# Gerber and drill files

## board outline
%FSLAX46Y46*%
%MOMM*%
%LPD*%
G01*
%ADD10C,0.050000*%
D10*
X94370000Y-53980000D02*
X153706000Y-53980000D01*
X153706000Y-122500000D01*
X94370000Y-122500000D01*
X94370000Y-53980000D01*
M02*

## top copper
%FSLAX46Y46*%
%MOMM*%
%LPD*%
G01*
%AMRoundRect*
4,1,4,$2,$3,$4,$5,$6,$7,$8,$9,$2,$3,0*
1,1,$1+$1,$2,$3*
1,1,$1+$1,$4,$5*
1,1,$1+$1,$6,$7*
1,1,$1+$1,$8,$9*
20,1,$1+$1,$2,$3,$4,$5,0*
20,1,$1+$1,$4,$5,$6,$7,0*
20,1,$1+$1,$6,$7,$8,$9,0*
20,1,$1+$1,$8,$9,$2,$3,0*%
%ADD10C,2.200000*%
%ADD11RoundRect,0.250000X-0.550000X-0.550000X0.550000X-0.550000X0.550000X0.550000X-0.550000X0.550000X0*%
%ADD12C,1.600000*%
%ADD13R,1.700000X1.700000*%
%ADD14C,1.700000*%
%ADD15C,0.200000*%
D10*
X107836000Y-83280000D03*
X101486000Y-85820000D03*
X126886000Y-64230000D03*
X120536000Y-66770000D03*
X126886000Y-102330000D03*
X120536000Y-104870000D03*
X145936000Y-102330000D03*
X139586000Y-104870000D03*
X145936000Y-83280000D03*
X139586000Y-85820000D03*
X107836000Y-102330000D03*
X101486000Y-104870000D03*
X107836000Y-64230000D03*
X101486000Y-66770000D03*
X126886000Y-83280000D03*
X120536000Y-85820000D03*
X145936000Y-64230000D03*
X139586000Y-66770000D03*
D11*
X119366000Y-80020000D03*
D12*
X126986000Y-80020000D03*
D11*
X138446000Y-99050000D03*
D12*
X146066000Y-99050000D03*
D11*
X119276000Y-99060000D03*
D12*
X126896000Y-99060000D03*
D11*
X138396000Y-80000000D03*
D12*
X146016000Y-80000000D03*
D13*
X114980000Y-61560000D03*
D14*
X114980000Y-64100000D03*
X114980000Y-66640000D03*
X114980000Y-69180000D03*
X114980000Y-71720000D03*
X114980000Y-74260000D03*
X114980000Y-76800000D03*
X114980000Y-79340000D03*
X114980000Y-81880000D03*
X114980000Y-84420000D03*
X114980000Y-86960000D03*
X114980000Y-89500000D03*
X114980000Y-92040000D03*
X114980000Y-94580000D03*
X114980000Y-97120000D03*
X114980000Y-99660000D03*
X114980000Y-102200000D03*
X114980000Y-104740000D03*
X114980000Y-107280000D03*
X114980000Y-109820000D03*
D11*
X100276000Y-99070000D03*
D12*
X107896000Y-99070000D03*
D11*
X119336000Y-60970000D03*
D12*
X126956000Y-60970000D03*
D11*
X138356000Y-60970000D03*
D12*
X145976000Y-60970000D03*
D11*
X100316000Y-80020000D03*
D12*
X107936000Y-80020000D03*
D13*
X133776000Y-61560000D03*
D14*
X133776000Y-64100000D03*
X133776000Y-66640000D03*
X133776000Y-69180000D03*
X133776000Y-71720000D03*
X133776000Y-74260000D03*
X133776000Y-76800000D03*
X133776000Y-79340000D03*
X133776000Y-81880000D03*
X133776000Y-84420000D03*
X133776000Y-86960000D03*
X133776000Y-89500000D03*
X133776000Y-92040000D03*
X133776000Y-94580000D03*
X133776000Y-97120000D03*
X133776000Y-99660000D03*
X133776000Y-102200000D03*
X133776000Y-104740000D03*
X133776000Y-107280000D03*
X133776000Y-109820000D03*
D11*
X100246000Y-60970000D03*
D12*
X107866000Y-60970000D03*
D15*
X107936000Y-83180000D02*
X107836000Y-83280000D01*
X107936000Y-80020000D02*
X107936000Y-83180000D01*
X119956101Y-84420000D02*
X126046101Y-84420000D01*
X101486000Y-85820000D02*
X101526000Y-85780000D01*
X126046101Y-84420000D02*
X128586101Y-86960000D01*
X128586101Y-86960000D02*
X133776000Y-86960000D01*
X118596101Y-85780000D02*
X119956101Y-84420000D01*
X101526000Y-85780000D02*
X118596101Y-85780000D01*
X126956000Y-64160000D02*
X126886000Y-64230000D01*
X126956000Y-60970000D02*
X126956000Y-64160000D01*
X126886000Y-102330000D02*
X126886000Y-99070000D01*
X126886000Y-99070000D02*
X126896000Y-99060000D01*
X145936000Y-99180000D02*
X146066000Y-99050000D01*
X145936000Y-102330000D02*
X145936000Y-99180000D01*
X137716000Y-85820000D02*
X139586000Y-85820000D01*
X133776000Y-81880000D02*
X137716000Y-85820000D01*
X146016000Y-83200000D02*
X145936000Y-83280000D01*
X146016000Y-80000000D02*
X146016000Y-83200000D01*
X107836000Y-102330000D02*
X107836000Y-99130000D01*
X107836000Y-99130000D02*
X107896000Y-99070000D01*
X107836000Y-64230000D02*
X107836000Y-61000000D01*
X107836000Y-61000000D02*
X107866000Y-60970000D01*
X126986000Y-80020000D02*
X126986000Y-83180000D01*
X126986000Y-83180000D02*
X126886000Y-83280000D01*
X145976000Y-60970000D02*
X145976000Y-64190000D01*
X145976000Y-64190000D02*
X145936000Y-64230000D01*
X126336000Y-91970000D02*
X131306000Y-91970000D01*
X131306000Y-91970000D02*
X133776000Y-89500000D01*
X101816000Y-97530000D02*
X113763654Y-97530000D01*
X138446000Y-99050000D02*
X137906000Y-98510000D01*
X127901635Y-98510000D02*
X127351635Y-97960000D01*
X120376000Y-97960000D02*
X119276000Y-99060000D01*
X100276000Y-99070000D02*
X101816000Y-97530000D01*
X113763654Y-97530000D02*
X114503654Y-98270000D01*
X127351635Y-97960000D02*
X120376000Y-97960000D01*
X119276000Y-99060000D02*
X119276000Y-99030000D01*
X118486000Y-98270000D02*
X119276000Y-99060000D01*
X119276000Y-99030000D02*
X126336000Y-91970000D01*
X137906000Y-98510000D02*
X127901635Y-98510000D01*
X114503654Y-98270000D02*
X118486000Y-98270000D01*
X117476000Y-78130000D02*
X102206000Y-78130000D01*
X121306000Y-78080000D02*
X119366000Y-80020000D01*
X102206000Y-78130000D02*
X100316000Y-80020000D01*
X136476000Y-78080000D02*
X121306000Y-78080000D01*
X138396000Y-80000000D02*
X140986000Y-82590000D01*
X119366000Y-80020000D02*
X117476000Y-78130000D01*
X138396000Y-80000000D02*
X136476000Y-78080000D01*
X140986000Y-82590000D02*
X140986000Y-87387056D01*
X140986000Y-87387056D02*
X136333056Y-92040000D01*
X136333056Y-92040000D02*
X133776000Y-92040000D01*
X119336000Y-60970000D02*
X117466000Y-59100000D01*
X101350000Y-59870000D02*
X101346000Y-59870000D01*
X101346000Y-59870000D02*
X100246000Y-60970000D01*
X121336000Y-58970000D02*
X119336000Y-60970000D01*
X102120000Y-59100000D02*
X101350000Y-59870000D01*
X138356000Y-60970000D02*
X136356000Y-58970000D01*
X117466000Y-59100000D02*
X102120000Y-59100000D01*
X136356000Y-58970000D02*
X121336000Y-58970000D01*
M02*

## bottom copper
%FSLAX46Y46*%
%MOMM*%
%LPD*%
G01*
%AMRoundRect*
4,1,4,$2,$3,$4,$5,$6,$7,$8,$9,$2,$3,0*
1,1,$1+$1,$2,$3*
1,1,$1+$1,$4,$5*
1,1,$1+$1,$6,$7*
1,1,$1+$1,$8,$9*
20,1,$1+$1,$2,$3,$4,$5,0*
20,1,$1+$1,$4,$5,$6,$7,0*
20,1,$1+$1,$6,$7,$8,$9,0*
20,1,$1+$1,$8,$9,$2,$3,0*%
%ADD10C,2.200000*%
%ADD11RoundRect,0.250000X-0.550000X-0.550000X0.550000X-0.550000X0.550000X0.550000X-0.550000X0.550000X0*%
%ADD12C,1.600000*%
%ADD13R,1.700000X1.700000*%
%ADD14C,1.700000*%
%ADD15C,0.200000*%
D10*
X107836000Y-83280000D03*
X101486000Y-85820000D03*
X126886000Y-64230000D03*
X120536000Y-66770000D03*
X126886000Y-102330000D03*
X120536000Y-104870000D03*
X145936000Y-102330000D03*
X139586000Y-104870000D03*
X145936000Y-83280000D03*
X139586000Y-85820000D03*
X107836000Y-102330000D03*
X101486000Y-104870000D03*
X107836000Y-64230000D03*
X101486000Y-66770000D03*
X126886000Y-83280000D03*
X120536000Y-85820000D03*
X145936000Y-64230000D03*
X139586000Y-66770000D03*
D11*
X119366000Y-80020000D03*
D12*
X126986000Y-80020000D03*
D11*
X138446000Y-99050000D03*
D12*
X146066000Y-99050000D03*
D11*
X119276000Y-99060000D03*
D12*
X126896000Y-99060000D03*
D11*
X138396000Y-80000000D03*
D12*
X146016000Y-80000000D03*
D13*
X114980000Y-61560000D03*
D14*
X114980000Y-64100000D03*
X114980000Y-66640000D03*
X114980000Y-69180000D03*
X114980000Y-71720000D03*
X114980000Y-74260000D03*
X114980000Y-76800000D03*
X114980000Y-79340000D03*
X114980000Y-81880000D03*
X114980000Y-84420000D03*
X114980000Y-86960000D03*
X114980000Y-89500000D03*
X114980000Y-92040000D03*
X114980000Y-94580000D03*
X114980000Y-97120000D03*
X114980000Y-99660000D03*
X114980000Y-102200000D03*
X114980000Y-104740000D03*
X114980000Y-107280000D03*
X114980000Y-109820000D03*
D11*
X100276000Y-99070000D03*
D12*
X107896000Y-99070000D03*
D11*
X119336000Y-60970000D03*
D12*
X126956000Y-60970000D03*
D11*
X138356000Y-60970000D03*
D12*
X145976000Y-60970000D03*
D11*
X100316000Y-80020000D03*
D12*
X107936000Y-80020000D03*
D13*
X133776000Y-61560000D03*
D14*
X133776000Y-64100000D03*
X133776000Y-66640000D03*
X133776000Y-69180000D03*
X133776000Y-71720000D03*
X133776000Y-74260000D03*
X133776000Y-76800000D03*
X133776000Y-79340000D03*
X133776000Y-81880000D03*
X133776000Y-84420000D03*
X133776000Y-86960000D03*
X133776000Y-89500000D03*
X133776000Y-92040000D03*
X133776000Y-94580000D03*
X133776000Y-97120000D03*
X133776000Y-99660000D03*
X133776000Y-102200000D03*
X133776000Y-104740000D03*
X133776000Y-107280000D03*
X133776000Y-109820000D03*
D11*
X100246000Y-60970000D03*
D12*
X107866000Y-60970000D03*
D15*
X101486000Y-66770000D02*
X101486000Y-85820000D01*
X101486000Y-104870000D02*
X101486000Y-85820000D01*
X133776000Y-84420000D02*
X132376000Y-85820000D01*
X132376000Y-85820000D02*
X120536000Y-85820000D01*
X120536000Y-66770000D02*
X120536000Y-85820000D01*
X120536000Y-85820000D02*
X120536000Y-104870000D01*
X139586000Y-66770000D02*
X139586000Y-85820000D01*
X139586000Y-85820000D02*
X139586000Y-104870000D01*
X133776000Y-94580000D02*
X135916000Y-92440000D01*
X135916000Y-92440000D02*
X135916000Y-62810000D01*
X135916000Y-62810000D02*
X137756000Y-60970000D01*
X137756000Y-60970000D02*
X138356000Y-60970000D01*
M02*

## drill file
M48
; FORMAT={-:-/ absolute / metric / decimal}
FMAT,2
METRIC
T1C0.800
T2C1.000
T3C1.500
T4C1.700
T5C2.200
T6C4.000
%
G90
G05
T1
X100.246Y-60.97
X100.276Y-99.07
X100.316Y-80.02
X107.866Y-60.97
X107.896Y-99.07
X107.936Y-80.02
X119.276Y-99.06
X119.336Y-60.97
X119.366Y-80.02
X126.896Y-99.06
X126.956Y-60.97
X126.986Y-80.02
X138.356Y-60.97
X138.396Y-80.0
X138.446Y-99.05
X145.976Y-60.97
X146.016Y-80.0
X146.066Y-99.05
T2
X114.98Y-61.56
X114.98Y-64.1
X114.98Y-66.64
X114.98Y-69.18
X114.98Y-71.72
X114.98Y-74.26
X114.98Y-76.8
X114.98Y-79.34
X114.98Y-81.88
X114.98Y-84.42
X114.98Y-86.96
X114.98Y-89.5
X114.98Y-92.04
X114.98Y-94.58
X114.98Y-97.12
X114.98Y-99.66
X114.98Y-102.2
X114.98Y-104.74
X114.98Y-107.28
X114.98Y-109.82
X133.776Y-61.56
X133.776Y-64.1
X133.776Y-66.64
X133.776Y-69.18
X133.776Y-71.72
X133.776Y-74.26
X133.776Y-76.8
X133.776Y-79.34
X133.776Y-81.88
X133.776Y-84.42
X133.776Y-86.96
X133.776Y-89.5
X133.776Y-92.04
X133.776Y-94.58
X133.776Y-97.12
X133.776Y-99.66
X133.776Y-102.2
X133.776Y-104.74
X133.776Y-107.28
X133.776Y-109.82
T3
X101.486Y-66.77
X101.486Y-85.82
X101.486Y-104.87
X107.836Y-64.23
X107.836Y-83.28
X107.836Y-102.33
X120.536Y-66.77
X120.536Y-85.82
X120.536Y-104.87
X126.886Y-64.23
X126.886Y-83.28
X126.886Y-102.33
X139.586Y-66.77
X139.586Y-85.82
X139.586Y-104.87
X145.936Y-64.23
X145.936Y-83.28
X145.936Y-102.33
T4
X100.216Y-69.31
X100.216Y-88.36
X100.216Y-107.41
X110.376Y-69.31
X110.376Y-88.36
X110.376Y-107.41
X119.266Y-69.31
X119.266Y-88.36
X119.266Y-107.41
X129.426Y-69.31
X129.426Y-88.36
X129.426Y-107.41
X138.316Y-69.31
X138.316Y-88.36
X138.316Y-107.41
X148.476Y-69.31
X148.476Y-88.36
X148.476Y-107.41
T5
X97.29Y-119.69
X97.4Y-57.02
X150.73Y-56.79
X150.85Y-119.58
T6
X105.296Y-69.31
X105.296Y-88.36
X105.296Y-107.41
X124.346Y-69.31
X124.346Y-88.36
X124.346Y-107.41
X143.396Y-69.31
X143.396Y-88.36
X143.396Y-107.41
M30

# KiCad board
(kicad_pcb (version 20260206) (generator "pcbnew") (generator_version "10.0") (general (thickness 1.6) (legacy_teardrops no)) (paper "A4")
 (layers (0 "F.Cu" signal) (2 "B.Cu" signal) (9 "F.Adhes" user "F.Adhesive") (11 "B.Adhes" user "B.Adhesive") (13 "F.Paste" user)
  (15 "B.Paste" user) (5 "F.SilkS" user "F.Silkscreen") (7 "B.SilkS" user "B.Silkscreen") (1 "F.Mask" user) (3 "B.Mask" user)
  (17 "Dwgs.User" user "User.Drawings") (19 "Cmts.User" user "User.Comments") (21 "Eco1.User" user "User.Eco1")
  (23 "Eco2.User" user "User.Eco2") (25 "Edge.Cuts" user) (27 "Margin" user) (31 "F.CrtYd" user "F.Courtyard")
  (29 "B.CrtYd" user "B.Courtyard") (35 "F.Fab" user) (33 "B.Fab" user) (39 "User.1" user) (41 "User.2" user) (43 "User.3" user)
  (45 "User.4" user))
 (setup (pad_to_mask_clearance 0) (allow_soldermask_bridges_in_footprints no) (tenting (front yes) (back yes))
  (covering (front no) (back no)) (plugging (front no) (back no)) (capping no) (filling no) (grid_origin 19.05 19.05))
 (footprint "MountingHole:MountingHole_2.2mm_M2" (layer "F.Cu") (at 150.73 56.79)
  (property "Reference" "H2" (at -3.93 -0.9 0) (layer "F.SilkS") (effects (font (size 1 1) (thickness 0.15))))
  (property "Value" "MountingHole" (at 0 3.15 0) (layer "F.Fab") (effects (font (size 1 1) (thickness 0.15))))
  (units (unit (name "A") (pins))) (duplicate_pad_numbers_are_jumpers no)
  (pad "" np_thru_hole circle (at 0 0) (size 2.2 2.2) (drill 2.2) (layers "*.Cu" "*.Mask")))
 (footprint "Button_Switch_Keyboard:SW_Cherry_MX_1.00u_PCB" (layer "F.Cu") (at 107.836 83.28)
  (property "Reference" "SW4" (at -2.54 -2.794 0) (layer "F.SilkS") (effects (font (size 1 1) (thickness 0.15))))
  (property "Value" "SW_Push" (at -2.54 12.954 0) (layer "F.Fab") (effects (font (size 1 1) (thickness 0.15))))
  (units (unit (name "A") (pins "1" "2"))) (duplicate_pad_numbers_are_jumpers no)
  (pad "" np_thru_hole circle (at -7.62 5.08) (size 1.7 1.7) (drill 1.7) (layers "*.Cu" "*.Mask"))
  (pad "" np_thru_hole circle (at -2.54 5.08) (size 4 4) (drill 4) (layers "*.Cu" "*.Mask"))
  (pad "" np_thru_hole circle (at 2.54 5.08) (size 1.7 1.7) (drill 1.7) (layers "*.Cu" "*.Mask"))
  (pad "1" thru_hole circle (at 0 0) (size 2.2 2.2) (drill 1.5) (layers "*.Cu" "*.Mask") (remove_unused_layers no) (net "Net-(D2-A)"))
  (pad "2" thru_hole circle (at -6.35 2.54) (size 2.2 2.2) (drill 1.5) (layers "*.Cu" "*.Mask") (remove_unused_layers no) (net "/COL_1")))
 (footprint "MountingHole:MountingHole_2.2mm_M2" (layer "F.Cu") (at 97.4 57.02)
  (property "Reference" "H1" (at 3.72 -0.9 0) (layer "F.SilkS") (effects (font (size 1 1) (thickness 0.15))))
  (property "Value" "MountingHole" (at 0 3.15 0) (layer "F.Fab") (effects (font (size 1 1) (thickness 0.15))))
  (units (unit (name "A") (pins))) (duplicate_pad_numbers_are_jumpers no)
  (pad "" np_thru_hole circle (at 0 0) (size 2.2 2.2) (drill 2.2) (layers "*.Cu" "*.Mask")))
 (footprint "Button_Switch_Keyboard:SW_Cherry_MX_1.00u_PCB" (layer "F.Cu") (at 126.886 64.23)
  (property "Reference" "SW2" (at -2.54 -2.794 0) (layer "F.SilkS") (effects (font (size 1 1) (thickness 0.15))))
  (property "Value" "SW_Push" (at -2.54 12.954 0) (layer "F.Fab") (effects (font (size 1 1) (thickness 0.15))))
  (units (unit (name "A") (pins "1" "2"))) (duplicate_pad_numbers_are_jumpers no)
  (pad "" np_thru_hole circle (at -7.62 5.08) (size 1.7 1.7) (drill 1.7) (layers "*.Cu" "*.Mask"))
  (pad "" np_thru_hole circle (at -2.54 5.08) (size 4 4) (drill 4) (layers "*.Cu" "*.Mask"))
  (pad "" np_thru_hole circle (at 2.54 5.08) (size 1.7 1.7) (drill 1.7) (layers "*.Cu" "*.Mask"))
  (pad "1" thru_hole circle (at 0 0) (size 2.2 2.2) (drill 1.5) (layers "*.Cu" "*.Mask") (remove_unused_layers no) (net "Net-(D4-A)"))
  (pad "2" thru_hole circle (at -6.35 2.54) (size 2.2 2.2) (drill 1.5) (layers "*.Cu" "*.Mask") (remove_unused_layers no) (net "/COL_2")))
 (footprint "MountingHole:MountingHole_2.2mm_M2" (layer "F.Cu") (at 97.29 119.69)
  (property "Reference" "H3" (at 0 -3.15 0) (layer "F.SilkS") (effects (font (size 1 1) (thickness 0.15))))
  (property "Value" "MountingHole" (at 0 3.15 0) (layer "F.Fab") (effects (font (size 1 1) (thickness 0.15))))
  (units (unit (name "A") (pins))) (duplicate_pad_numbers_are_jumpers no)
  (pad "" np_thru_hole circle (at 0 0) (size 2.2 2.2) (drill 2.2) (layers "*.Cu" "*.Mask")))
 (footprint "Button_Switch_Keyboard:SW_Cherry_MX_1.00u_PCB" (layer "F.Cu") (at 126.886 102.33)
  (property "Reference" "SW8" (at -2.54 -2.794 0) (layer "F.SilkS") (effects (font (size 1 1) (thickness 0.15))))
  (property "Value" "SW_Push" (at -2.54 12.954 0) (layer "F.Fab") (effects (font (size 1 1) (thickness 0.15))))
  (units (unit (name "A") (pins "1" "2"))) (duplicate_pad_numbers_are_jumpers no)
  (pad "" np_thru_hole circle (at -7.62 5.08) (size 1.7 1.7) (drill 1.7) (layers "*.Cu" "*.Mask"))
  (pad "" np_thru_hole circle (at -2.54 5.08) (size 4 4) (drill 4) (layers "*.Cu" "*.Mask"))
  (pad "" np_thru_hole circle (at 2.54 5.08) (size 1.7 1.7) (drill 1.7) (layers "*.Cu" "*.Mask"))
  (pad "1" thru_hole circle (at 0 0) (size 2.2 2.2) (drill 1.5) (layers "*.Cu" "*.Mask") (remove_unused_layers no) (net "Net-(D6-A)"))
  (pad "2" thru_hole circle (at -6.35 2.54) (size 2.2 2.2) (drill 1.5) (layers "*.Cu" "*.Mask") (remove_unused_layers no) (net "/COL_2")))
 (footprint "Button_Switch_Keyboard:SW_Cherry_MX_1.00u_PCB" (layer "F.Cu") (at 145.936 102.33)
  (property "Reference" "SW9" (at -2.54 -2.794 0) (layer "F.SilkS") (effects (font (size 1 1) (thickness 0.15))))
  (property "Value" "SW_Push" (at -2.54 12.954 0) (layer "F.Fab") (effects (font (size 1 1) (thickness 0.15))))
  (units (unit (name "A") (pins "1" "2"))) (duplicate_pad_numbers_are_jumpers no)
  (pad "" np_thru_hole circle (at -7.62 5.08) (size 1.7 1.7) (drill 1.7) (layers "*.Cu" "*.Mask"))
  (pad "" np_thru_hole circle (at -2.54 5.08) (size 4 4) (drill 4) (layers "*.Cu" "*.Mask"))
  (pad "" np_thru_hole circle (at 2.54 5.08) (size 1.7 1.7) (drill 1.7) (layers "*.Cu" "*.Mask"))
  (pad "1" thru_hole circle (at 0 0) (size 2.2 2.2) (drill 1.5) (layers "*.Cu" "*.Mask") (remove_unused_layers no) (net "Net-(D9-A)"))
  (pad "2" thru_hole circle (at -6.35 2.54) (size 2.2 2.2) (drill 1.5) (layers "*.Cu" "*.Mask") (remove_unused_layers no) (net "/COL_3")))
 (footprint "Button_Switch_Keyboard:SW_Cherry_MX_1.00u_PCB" (layer "F.Cu") (at 145.936 83.28)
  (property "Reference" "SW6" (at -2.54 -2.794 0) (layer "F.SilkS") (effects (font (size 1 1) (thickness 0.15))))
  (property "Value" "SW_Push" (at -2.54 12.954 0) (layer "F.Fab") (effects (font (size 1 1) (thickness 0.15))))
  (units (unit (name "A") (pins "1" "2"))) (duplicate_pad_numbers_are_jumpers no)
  (pad "" np_thru_hole circle (at -7.62 5.08) (size 1.7 1.7) (drill 1.7) (layers "*.Cu" "*.Mask"))
  (pad "" np_thru_hole circle (at -2.54 5.08) (size 4 4) (drill 4) (layers "*.Cu" "*.Mask"))
  (pad "" np_thru_hole circle (at 2.54 5.08) (size 1.7 1.7) (drill 1.7) (layers "*.Cu" "*.Mask"))
  (pad "1" thru_hole circle (at 0 0) (size 2.2 2.2) (drill 1.5) (layers "*.Cu" "*.Mask") (remove_unused_layers no) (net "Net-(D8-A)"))
  (pad "2" thru_hole circle (at -6.35 2.54) (size 2.2 2.2) (drill 1.5) (layers "*.Cu" "*.Mask") (remove_unused_layers no) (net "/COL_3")))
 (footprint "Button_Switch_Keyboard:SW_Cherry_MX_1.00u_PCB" (layer "F.Cu") (at 107.836 102.33)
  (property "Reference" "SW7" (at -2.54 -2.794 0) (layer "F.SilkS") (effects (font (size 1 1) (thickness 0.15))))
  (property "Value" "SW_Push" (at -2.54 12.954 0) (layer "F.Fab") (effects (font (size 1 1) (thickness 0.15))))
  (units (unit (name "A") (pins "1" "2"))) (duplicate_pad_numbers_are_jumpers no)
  (pad "" np_thru_hole circle (at -7.62 5.08) (size 1.7 1.7) (drill 1.7) (layers "*.Cu" "*.Mask"))
  (pad "" np_thru_hole circle (at -2.54 5.08) (size 4 4) (drill 4) (layers "*.Cu" "*.Mask"))
  (pad "" np_thru_hole circle (at 2.54 5.08) (size 1.7 1.7) (drill 1.7) (layers "*.Cu" "*.Mask"))
  (pad "1" thru_hole circle (at 0 0) (size 2.2 2.2) (drill 1.5) (layers "*.Cu" "*.Mask") (remove_unused_layers no) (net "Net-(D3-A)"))
  (pad "2" thru_hole circle (at -6.35 2.54) (size 2.2 2.2) (drill 1.5) (layers "*.Cu" "*.Mask") (remove_unused_layers no) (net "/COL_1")))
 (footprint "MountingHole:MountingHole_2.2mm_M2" (layer "F.Cu") (at 150.85 119.58)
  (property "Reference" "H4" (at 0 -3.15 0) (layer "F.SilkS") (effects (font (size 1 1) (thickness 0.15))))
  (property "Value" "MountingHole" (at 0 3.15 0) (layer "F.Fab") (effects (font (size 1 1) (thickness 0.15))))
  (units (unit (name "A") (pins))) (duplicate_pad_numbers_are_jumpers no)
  (pad "" np_thru_hole circle (at 0 0) (size 2.2 2.2) (drill 2.2) (layers "*.Cu" "*.Mask")))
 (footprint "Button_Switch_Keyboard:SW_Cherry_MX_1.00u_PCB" (layer "F.Cu") (at 107.836 64.23)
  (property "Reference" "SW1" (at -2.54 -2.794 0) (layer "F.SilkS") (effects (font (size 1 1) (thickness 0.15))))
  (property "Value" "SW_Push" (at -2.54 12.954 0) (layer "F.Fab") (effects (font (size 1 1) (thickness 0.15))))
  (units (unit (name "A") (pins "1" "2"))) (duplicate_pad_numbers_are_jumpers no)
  (pad "" np_thru_hole circle (at -7.62 5.08) (size 1.7 1.7) (drill 1.7) (layers "*.Cu" "*.Mask"))
  (pad "" np_thru_hole circle (at -2.54 5.08) (size 4 4) (drill 4) (layers "*.Cu" "*.Mask"))
  (pad "" np_thru_hole circle (at 2.54 5.08) (size 1.7 1.7) (drill 1.7) (layers "*.Cu" "*.Mask"))
  (pad "1" thru_hole circle (at 0 0) (size 2.2 2.2) (drill 1.5) (layers "*.Cu" "*.Mask") (remove_unused_layers no) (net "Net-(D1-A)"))
  (pad "2" thru_hole circle (at -6.35 2.54) (size 2.2 2.2) (drill 1.5) (layers "*.Cu" "*.Mask") (remove_unused_layers no) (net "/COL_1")))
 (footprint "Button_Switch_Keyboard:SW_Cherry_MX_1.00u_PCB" (layer "F.Cu") (at 126.886 83.28)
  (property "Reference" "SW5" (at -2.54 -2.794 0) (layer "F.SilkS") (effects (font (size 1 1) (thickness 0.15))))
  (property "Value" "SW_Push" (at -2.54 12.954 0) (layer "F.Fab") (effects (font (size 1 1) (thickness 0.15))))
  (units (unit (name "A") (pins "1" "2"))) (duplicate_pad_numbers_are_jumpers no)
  (pad "" np_thru_hole circle (at -7.62 5.08) (size 1.7 1.7) (drill 1.7) (layers "*.Cu" "*.Mask"))
  (pad "" np_thru_hole circle (at -2.54 5.08) (size 4 4) (drill 4) (layers "*.Cu" "*.Mask"))
  (pad "" np_thru_hole circle (at 2.54 5.08) (size 1.7 1.7) (drill 1.7) (layers "*.Cu" "*.Mask"))
  (pad "1" thru_hole circle (at 0 0) (size 2.2 2.2) (drill 1.5) (layers "*.Cu" "*.Mask") (remove_unused_layers no) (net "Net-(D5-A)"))
  (pad "2" thru_hole circle (at -6.35 2.54) (size 2.2 2.2) (drill 1.5) (layers "*.Cu" "*.Mask") (remove_unused_layers no) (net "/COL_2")))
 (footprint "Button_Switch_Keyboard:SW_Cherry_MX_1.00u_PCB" (layer "F.Cu") (at 145.936 64.23)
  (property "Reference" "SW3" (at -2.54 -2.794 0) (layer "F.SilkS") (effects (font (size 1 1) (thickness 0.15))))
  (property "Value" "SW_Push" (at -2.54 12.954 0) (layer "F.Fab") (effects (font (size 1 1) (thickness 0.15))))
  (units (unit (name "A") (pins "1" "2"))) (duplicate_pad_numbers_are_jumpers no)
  (pad "" np_thru_hole circle (at -7.62 5.08) (size 1.7 1.7) (drill 1.7) (layers "*.Cu" "*.Mask"))
  (pad "" np_thru_hole circle (at -2.54 5.08) (size 4 4) (drill 4) (layers "*.Cu" "*.Mask"))
  (pad "" np_thru_hole circle (at 2.54 5.08) (size 1.7 1.7) (drill 1.7) (layers "*.Cu" "*.Mask"))
  (pad "1" thru_hole circle (at 0 0) (size 2.2 2.2) (drill 1.5) (layers "*.Cu" "*.Mask") (remove_unused_layers no) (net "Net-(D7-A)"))
  (pad "2" thru_hole circle (at -6.35 2.54) (size 2.2 2.2) (drill 1.5) (layers "*.Cu" "*.Mask") (remove_unused_layers no) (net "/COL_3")))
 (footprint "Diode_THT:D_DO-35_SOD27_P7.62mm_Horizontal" (layer "B.Cu") (at 119.366 80.02)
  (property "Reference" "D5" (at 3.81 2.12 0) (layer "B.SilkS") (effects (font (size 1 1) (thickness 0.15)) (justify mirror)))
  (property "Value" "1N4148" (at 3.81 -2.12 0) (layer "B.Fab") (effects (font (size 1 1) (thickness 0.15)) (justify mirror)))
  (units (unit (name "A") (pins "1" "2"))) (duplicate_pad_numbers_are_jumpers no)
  (pad "1" thru_hole roundrect (at 0 0) (size 1.6 1.6) (drill 0.8) (layers "*.Cu" "*.Mask") (remove_unused_layers no)
   (roundrect_rratio 0.15625) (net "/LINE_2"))
  (pad "2" thru_hole circle (at 7.62 0) (size 1.6 1.6) (drill 0.8) (layers "*.Cu" "*.Mask") (remove_unused_layers no) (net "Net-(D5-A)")))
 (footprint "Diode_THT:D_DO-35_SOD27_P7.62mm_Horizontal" (layer "B.Cu") (at 138.446 99.05)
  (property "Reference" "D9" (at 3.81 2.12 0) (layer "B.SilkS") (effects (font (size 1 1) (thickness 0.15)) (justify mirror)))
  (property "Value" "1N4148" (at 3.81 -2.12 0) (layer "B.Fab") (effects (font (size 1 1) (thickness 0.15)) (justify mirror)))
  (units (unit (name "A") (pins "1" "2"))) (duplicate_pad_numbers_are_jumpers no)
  (pad "1" thru_hole roundrect (at 0 0) (size 1.6 1.6) (drill 0.8) (layers "*.Cu" "*.Mask") (remove_unused_layers no)
   (roundrect_rratio 0.15625) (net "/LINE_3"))
  (pad "2" thru_hole circle (at 7.62 0) (size 1.6 1.6) (drill 0.8) (layers "*.Cu" "*.Mask") (remove_unused_layers no) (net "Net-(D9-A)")))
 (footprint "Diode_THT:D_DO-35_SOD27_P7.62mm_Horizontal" (layer "B.Cu") (at 119.276 99.06)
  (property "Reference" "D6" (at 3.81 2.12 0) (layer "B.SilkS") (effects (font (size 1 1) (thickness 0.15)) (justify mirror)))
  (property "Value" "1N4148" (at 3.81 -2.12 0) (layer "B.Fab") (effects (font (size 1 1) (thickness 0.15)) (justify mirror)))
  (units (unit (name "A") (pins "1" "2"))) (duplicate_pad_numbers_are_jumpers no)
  (pad "1" thru_hole roundrect (at 0 0) (size 1.6 1.6) (drill 0.8) (layers "*.Cu" "*.Mask") (remove_unused_layers no)
   (roundrect_rratio 0.15625) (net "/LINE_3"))
  (pad "2" thru_hole circle (at 7.62 0) (size 1.6 1.6) (drill 0.8) (layers "*.Cu" "*.Mask") (remove_unused_layers no) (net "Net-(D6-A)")))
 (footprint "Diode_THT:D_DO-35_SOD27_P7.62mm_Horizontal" (layer "B.Cu") (at 138.396 80)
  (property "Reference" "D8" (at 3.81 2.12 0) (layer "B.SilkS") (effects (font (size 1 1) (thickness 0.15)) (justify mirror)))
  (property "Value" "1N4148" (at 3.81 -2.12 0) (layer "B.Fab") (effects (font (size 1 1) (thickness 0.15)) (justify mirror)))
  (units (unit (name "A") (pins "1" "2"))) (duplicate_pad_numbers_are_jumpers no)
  (pad "1" thru_hole roundrect (at 0 0) (size 1.6 1.6) (drill 0.8) (layers "*.Cu" "*.Mask") (remove_unused_layers no)
   (roundrect_rratio 0.15625) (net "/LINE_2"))
  (pad "2" thru_hole circle (at 7.62 0) (size 1.6 1.6) (drill 0.8) (layers "*.Cu" "*.Mask") (remove_unused_layers no) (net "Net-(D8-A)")))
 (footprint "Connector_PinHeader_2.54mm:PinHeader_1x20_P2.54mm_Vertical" (layer "B.Cu") (at 114.98 61.56 180)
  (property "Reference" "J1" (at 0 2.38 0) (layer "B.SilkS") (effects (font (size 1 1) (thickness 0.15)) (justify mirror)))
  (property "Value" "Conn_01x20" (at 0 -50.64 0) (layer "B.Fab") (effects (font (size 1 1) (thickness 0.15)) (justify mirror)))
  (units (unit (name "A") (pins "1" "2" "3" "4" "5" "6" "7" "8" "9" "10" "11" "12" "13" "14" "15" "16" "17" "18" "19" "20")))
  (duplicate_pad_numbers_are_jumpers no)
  (pad "1" thru_hole rect (at 0 0 180) (size 1.7 1.7) (drill 1) (layers "*.Cu" "*.Mask") (remove_unused_layers no)
   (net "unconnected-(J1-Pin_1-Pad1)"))
  (pad "2" thru_hole circle (at 0 -2.54 180) (size 1.7 1.7) (drill 1) (layers "*.Cu" "*.Mask") (remove_unused_layers no)
   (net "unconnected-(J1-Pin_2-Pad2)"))
  (pad "3" thru_hole circle (at 0 -5.08 180) (size 1.7 1.7) (drill 1) (layers "*.Cu" "*.Mask") (remove_unused_layers no)
   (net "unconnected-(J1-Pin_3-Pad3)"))
  (pad "4" thru_hole circle (at 0 -7.62 180) (size 1.7 1.7) (drill 1) (layers "*.Cu" "*.Mask") (remove_unused_layers no)
   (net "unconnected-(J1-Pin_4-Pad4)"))
  (pad "5" thru_hole circle (at 0 -10.16 180) (size 1.7 1.7) (drill 1) (layers "*.Cu" "*.Mask") (remove_unused_layers no)
   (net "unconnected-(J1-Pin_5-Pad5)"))
  (pad "6" thru_hole circle (at 0 -12.7 180) (size 1.7 1.7) (drill 1) (layers "*.Cu" "*.Mask") (remove_unused_layers no)
   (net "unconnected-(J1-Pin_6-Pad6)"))
  (pad "7" thru_hole circle (at 0 -15.24 180) (size 1.7 1.7) (drill 1) (layers "*.Cu" "*.Mask") (remove_unused_layers no)
   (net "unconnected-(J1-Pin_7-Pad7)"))
  (pad "8" thru_hole circle (at 0 -17.78 180) (size 1.7 1.7) (drill 1) (layers "*.Cu" "*.Mask") (remove_unused_layers no)
   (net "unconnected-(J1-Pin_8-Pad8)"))
  (pad "9" thru_hole circle (at 0 -20.32 180) (size 1.7 1.7) (drill 1) (layers "*.Cu" "*.Mask") (remove_unused_layers no)
   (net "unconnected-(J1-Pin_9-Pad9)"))
  (pad "10" thru_hole circle (at 0 -22.86 180) (size 1.7 1.7) (drill 1) (layers "*.Cu" "*.Mask") (remove_unused_layers no)
   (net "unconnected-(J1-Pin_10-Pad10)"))
  (pad "11" thru_hole circle (at 0 -25.4 180) (size 1.7 1.7) (drill 1) (layers "*.Cu" "*.Mask") (remove_unused_layers no)
   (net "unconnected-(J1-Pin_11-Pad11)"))
  (pad "12" thru_hole circle (at 0 -27.94 180) (size 1.7 1.7) (drill 1) (layers "*.Cu" "*.Mask") (remove_unused_layers no)
   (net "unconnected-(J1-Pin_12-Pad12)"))
  (pad "13" thru_hole circle (at 0 -30.48 180) (size 1.7 1.7) (drill 1) (layers "*.Cu" "*.Mask") (remove_unused_layers no)
   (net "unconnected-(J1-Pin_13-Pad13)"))
  (pad "14" thru_hole circle (at 0 -33.02 180) (size 1.7 1.7) (drill 1) (layers "*.Cu" "*.Mask") (remove_unused_layers no)
   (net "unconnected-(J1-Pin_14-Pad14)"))
  (pad "15" thru_hole circle (at 0 -35.56 180) (size 1.7 1.7) (drill 1) (layers "*.Cu" "*.Mask") (remove_unused_layers no)
   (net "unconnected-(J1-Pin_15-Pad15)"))
  (pad "16" thru_hole circle (at 0 -38.1 180) (size 1.7 1.7) (drill 1) (layers "*.Cu" "*.Mask") (remove_unused_layers no)
   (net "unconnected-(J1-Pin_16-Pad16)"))
  (pad "17" thru_hole circle (at 0 -40.64 180) (size 1.7 1.7) (drill 1) (layers "*.Cu" "*.Mask") (remove_unused_layers no)
   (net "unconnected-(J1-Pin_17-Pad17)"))
  (pad "18" thru_hole circle (at 0 -43.18 180) (size 1.7 1.7) (drill 1) (layers "*.Cu" "*.Mask") (remove_unused_layers no)
   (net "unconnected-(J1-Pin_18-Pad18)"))
  (pad "19" thru_hole circle (at 0 -45.72 180) (size 1.7 1.7) (drill 1) (layers "*.Cu" "*.Mask") (remove_unused_layers no)
   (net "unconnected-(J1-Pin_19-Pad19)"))
  (pad "20" thru_hole circle (at 0 -48.26 180) (size 1.7 1.7) (drill 1) (layers "*.Cu" "*.Mask") (remove_unused_layers no)
   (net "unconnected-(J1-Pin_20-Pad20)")))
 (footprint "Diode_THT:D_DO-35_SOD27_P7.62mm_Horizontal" (layer "B.Cu") (at 100.276 99.07)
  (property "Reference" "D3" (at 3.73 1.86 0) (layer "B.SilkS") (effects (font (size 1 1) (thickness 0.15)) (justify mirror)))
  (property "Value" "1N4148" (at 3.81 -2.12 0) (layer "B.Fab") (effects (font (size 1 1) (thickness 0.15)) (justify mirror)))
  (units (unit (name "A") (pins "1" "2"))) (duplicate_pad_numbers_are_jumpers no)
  (pad "1" thru_hole roundrect (at 0 0) (size 1.6 1.6) (drill 0.8) (layers "*.Cu" "*.Mask") (remove_unused_layers no)
   (roundrect_rratio 0.15625) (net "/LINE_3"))
  (pad "2" thru_hole circle (at 7.62 0) (size 1.6 1.6) (drill 0.8) (layers "*.Cu" "*.Mask") (remove_unused_layers no) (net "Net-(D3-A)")))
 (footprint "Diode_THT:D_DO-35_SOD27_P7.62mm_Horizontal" (layer "B.Cu") (at 119.336 60.97)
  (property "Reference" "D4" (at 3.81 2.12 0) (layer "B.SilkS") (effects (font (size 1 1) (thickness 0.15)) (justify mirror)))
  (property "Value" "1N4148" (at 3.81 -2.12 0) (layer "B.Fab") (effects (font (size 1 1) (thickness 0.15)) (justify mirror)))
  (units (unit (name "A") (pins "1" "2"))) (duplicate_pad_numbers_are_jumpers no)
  (pad "1" thru_hole roundrect (at 0 0) (size 1.6 1.6) (drill 0.8) (layers "*.Cu" "*.Mask") (remove_unused_layers no)
   (roundrect_rratio 0.15625) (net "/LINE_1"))
  (pad "2" thru_hole circle (at 7.62 0) (size 1.6 1.6) (drill 0.8) (layers "*.Cu" "*.Mask") (remove_unused_layers no) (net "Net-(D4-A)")))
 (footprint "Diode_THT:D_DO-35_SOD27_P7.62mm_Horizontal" (layer "B.Cu") (at 138.356 60.97)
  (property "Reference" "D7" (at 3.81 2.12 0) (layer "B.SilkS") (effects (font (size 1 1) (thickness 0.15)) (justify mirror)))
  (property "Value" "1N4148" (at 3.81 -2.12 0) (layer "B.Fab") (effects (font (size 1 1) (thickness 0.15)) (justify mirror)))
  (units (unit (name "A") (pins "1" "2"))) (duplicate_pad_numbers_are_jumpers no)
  (pad "1" thru_hole roundrect (at 0 0) (size 1.6 1.6) (drill 0.8) (layers "*.Cu" "*.Mask") (remove_unused_layers no)
   (roundrect_rratio 0.15625) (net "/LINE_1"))
  (pad "2" thru_hole circle (at 7.62 0) (size 1.6 1.6) (drill 0.8) (layers "*.Cu" "*.Mask") (remove_unused_layers no) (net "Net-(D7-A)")))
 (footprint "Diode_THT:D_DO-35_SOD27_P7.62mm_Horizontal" (layer "B.Cu") (at 100.316 80.02)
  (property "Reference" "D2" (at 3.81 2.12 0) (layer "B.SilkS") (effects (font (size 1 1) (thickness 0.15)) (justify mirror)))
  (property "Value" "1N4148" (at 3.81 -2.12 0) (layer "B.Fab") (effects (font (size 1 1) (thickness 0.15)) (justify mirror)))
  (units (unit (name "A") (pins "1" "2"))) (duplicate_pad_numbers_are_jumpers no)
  (pad "1" thru_hole roundrect (at 0 0) (size 1.6 1.6) (drill 0.8) (layers "*.Cu" "*.Mask") (remove_unused_layers no)
   (roundrect_rratio 0.15625) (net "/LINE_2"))
  (pad "2" thru_hole circle (at 7.62 0) (size 1.6 1.6) (drill 0.8) (layers "*.Cu" "*.Mask") (remove_unused_layers no) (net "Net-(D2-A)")))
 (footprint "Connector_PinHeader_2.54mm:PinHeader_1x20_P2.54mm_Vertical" (layer "B.Cu") (at 133.776 61.56 180)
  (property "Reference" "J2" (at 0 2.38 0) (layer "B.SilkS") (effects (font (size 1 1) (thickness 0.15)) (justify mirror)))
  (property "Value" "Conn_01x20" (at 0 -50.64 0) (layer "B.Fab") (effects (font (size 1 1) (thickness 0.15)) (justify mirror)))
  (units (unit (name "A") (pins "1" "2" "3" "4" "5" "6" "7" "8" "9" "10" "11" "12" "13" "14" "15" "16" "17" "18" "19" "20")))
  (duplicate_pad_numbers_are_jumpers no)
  (pad "1" thru_hole rect (at 0 0 180) (size 1.7 1.7) (drill 1) (layers "*.Cu" "*.Mask") (remove_unused_layers no)
   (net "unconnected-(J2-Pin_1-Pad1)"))
  (pad "2" thru_hole circle (at 0 -2.54 180) (size 1.7 1.7) (drill 1) (layers "*.Cu" "*.Mask") (remove_unused_layers no)
   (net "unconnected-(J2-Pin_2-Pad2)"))
  (pad "3" thru_hole circle (at 0 -5.08 180) (size 1.7 1.7) (drill 1) (layers "*.Cu" "*.Mask") (remove_unused_layers no)
   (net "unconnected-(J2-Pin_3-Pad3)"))
  (pad "4" thru_hole circle (at 0 -7.62 180) (size 1.7 1.7) (drill 1) (layers "*.Cu" "*.Mask") (remove_unused_layers no)
   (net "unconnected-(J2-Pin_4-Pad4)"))
  (pad "5" thru_hole circle (at 0 -10.16 180) (size 1.7 1.7) (drill 1) (layers "*.Cu" "*.Mask") (remove_unused_layers no)
   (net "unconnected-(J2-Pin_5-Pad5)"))
  (pad "6" thru_hole circle (at 0 -12.7 180) (size 1.7 1.7) (drill 1) (layers "*.Cu" "*.Mask") (remove_unused_layers no)
   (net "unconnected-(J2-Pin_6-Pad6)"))
  (pad "7" thru_hole circle (at 0 -15.24 180) (size 1.7 1.7) (drill 1) (layers "*.Cu" "*.Mask") (remove_unused_layers no)
   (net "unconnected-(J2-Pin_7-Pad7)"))
  (pad "8" thru_hole circle (at 0 -17.78 180) (size 1.7 1.7) (drill 1) (layers "*.Cu" "*.Mask") (remove_unused_layers no)
   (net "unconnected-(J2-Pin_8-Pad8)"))
  (pad "9" thru_hole circle (at 0 -20.32 180) (size 1.7 1.7) (drill 1) (layers "*.Cu" "*.Mask") (remove_unused_layers no) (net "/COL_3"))
  (pad "10" thru_hole circle (at 0 -22.86 180) (size 1.7 1.7) (drill 1) (layers "*.Cu" "*.Mask") (remove_unused_layers no) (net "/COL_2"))
  (pad "11" thru_hole circle (at 0 -25.4 180) (size 1.7 1.7) (drill 1) (layers "*.Cu" "*.Mask") (remove_unused_layers no) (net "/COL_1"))
  (pad "12" thru_hole circle (at 0 -27.94 180) (size 1.7 1.7) (drill 1) (layers "*.Cu" "*.Mask") (remove_unused_layers no) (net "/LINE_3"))
  (pad "13" thru_hole circle (at 0 -30.48 180) (size 1.7 1.7) (drill 1) (layers "*.Cu" "*.Mask") (remove_unused_layers no) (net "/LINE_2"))
  (pad "14" thru_hole circle (at 0 -33.02 180) (size 1.7 1.7) (drill 1) (layers "*.Cu" "*.Mask") (remove_unused_layers no) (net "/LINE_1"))
  (pad "15" thru_hole circle (at 0 -35.56 180) (size 1.7 1.7) (drill 1) (layers "*.Cu" "*.Mask") (remove_unused_layers no)
   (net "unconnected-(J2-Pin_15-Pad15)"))
  (pad "16" thru_hole circle (at 0 -38.1 180) (size 1.7 1.7) (drill 1) (layers "*.Cu" "*.Mask") (remove_unused_layers no)
   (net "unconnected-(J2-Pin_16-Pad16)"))
  (pad "17" thru_hole circle (at 0 -40.64 180) (size 1.7 1.7) (drill 1) (layers "*.Cu" "*.Mask") (remove_unused_layers no)
   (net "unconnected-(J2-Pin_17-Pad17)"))
  (pad "18" thru_hole circle (at 0 -43.18 180) (size 1.7 1.7) (drill 1) (layers "*.Cu" "*.Mask") (remove_unused_layers no)
   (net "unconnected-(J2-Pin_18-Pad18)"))
  (pad "19" thru_hole circle (at 0 -45.72 180) (size 1.7 1.7) (drill 1) (layers "*.Cu" "*.Mask") (remove_unused_layers no)
   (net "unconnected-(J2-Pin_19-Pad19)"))
  (pad "20" thru_hole circle (at 0 -48.26 180) (size 1.7 1.7) (drill 1) (layers "*.Cu" "*.Mask") (remove_unused_layers no)
   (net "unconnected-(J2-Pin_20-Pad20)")))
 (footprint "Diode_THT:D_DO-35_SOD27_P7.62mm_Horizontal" (layer "B.Cu") (at 100.246 60.97)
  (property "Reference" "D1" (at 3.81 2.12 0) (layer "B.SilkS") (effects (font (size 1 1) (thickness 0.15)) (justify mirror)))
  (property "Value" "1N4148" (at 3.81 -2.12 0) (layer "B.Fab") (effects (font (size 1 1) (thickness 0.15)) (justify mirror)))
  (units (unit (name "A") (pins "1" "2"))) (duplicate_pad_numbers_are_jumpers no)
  (pad "1" thru_hole roundrect (at 0 0) (size 1.6 1.6) (drill 0.8) (layers "*.Cu" "*.Mask") (remove_unused_layers no)
   (roundrect_rratio 0.15625) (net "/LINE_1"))
  (pad "2" thru_hole circle (at 7.62 0) (size 1.6 1.6) (drill 0.8) (layers "*.Cu" "*.Mask") (remove_unused_layers no) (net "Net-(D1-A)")))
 (gr_rect (start 94.37 53.98) (end 153.706 122.5) (stroke (width 0.05) (type default)) (fill no) (layer "Edge.Cuts"))
 (segment (start 107.936 83.18) (end 107.836 83.28) (width 0.2) (layer "F.Cu") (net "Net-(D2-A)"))
 (segment (start 107.936 80.02) (end 107.936 83.18) (width 0.2) (layer "F.Cu") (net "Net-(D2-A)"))
 (segment (start 119.956101 84.42) (end 126.046101 84.42) (width 0.2) (layer "F.Cu") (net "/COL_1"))
 (segment (start 101.486 85.82) (end 101.526 85.78) (width 0.2) (layer "F.Cu") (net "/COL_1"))
 (segment (start 126.046101 84.42) (end 128.586101 86.96) (width 0.2) (layer "F.Cu") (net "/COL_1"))
 (segment (start 128.586101 86.96) (end 133.776 86.96) (width 0.2) (layer "F.Cu") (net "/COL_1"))
 (segment (start 118.596101 85.78) (end 119.956101 84.42) (width 0.2) (layer "F.Cu") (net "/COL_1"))
 (segment (start 101.526 85.78) (end 118.596101 85.78) (width 0.2) (layer "F.Cu") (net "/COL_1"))
 (segment (start 101.486 66.77) (end 101.486 85.82) (width 0.2) (layer "B.Cu") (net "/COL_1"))
 (segment (start 101.486 104.87) (end 101.486 85.82) (width 0.2) (layer "B.Cu") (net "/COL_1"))
 (segment (start 126.956 64.16) (end 126.886 64.23) (width 0.2) (layer "F.Cu") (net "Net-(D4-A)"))
 (segment (start 126.956 60.97) (end 126.956 64.16) (width 0.2) (layer "F.Cu") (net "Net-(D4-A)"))
 (segment (start 133.776 84.42) (end 132.376 85.82) (width 0.2) (layer "B.Cu") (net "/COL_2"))
 (segment (start 132.376 85.82) (end 120.536 85.82) (width 0.2) (layer "B.Cu") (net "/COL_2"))
 (segment (start 120.536 66.77) (end 120.536 85.82) (width 0.2) (layer "B.Cu") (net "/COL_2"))
 (segment (start 120.536 85.82) (end 120.536 104.87) (width 0.2) (layer "B.Cu") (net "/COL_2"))
 (segment (start 126.886 102.33) (end 126.886 99.07) (width 0.2) (layer "F.Cu") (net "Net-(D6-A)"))
 (segment (start 126.886 99.07) (end 126.896 99.06) (width 0.2) (layer "F.Cu") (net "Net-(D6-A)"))
 (segment (start 145.936 99.18) (end 146.066 99.05) (width 0.2) (layer "F.Cu") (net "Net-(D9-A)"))
 (segment (start 145.936 102.33) (end 145.936 99.18) (width 0.2) (layer "F.Cu") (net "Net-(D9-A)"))
 (segment (start 137.716 85.82) (end 139.586 85.82) (width 0.2) (layer "F.Cu") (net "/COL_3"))
 (segment (start 133.776 81.88) (end 137.716 85.82) (width 0.2) (layer "F.Cu") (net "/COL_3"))
 (segment (start 139.586 66.77) (end 139.586 85.82) (width 0.2) (layer "B.Cu") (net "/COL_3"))
 (segment (start 139.586 85.82) (end 139.586 104.87) (width 0.2) (layer "B.Cu") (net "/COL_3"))
 (segment (start 146.016 83.2) (end 145.936 83.28) (width 0.2) (layer "F.Cu") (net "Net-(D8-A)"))
 (segment (start 146.016 80) (end 146.016 83.2) (width 0.2) (layer "F.Cu") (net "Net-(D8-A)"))
 (segment (start 107.836 102.33) (end 107.836 99.13) (width 0.2) (layer "F.Cu") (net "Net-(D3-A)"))
 (segment (start 107.836 99.13) (end 107.896 99.07) (width 0.2) (layer "F.Cu") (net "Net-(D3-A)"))
 (segment (start 107.836 64.23) (end 107.836 61) (width 0.2) (layer "F.Cu") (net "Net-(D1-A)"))
 (segment (start 107.836 61) (end 107.866 60.97) (width 0.2) (layer "F.Cu") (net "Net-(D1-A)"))
 (segment (start 126.986 80.02) (end 126.986 83.18) (width 0.2) (layer "F.Cu") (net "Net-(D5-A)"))
 (segment (start 126.986 83.18) (end 126.886 83.28) (width 0.2) (layer "F.Cu") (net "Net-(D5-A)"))
 (segment (start 145.976 60.97) (end 145.976 64.19) (width 0.2) (layer "F.Cu") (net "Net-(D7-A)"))
 (segment (start 145.976 64.19) (end 145.936 64.23) (width 0.2) (layer "F.Cu") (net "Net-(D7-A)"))
 (segment (start 126.336 91.97) (end 131.306 91.97) (width 0.2) (layer "F.Cu") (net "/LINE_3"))
 (segment (start 131.306 91.97) (end 133.776 89.5) (width 0.2) (layer "F.Cu") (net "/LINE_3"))
 (segment (start 101.816 97.53) (end 113.763654 97.53) (width 0.2) (layer "F.Cu") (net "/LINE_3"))
 (segment (start 138.446 99.05) (end 137.906 98.51) (width 0.2) (layer "F.Cu") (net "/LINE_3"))
 (segment (start 127.901635 98.51) (end 127.351635 97.96) (width 0.2) (layer "F.Cu") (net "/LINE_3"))
 (segment (start 120.376 97.96) (end 119.276 99.06) (width 0.2) (layer "F.Cu") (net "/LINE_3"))
 (segment (start 100.276 99.07) (end 101.816 97.53) (width 0.2) (layer "F.Cu") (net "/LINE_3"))
 (segment (start 113.763654 97.53) (end 114.503654 98.27) (width 0.2) (layer "F.Cu") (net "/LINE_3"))
 (segment (start 127.351635 97.96) (end 120.376 97.96) (width 0.2) (layer "F.Cu") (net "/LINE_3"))
 (segment (start 119.276 99.06) (end 119.276 99.03) (width 0.2) (layer "F.Cu") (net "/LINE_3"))
 (segment (start 118.486 98.27) (end 119.276 99.06) (width 0.2) (layer "F.Cu") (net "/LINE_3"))
 (segment (start 119.276 99.03) (end 126.336 91.97) (width 0.2) (layer "F.Cu") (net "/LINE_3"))
 (segment (start 137.906 98.51) (end 127.901635 98.51) (width 0.2) (layer "F.Cu") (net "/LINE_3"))
 (segment (start 114.503654 98.27) (end 118.486 98.27) (width 0.2) (layer "F.Cu") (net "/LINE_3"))
 (segment (start 117.476 78.13) (end 102.206 78.13) (width 0.2) (layer "F.Cu") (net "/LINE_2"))
 (segment (start 121.306 78.08) (end 119.366 80.02) (width 0.2) (layer "F.Cu") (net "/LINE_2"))
 (segment (start 102.206 78.13) (end 100.316 80.02) (width 0.2) (layer "F.Cu") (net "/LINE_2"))
 (segment (start 136.476 78.08) (end 121.306 78.08) (width 0.2) (layer "F.Cu") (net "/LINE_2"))
 (segment (start 138.396 80) (end 140.986 82.59) (width 0.2) (layer "F.Cu") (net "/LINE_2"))
 (segment (start 119.366 80.02) (end 117.476 78.13) (width 0.2) (layer "F.Cu") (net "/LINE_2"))
 (segment (start 138.396 80) (end 136.476 78.08) (width 0.2) (layer "F.Cu") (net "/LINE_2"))
 (segment (start 140.986 82.59) (end 140.986 87.387056) (width 0.2) (layer "F.Cu") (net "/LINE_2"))
 (segment (start 140.986 87.387056) (end 136.333056 92.04) (width 0.2) (layer "F.Cu") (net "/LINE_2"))
 (segment (start 136.333056 92.04) (end 133.776 92.04) (width 0.2) (layer "F.Cu") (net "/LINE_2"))
 (segment (start 119.336 60.97) (end 117.466 59.1) (width 0.2) (layer "F.Cu") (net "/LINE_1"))
 (segment (start 101.35 59.87) (end 101.346 59.87) (width 0.2) (layer "F.Cu") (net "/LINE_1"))
 (segment (start 101.346 59.87) (end 100.246 60.97) (width 0.2) (layer "F.Cu") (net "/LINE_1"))
 (segment (start 121.336 58.97) (end 119.336 60.97) (width 0.2) (layer "F.Cu") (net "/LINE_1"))
 (segment (start 102.12 59.1) (end 101.35 59.87) (width 0.2) (layer "F.Cu") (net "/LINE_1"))
 (segment (start 138.356 60.97) (end 136.356 58.97) (width 0.2) (layer "F.Cu") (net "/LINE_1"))
 (segment (start 117.466 59.1) (end 102.12 59.1) (width 0.2) (layer "F.Cu") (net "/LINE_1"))
 (segment (start 136.356 58.97) (end 121.336 58.97) (width 0.2) (layer "F.Cu") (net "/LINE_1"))
 (segment (start 133.776 94.58) (end 135.916 92.44) (width 0.2) (layer "B.Cu") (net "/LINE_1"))
 (segment (start 135.916 92.44) (end 135.916 62.81) (width 0.2) (layer "B.Cu") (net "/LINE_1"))
 (segment (start 135.916 62.81) (end 137.756 60.97) (width 0.2) (layer "B.Cu") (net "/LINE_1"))
 (segment (start 137.756 60.97) (end 138.356 60.97) (width 0.2) (layer "B.Cu") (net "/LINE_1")))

